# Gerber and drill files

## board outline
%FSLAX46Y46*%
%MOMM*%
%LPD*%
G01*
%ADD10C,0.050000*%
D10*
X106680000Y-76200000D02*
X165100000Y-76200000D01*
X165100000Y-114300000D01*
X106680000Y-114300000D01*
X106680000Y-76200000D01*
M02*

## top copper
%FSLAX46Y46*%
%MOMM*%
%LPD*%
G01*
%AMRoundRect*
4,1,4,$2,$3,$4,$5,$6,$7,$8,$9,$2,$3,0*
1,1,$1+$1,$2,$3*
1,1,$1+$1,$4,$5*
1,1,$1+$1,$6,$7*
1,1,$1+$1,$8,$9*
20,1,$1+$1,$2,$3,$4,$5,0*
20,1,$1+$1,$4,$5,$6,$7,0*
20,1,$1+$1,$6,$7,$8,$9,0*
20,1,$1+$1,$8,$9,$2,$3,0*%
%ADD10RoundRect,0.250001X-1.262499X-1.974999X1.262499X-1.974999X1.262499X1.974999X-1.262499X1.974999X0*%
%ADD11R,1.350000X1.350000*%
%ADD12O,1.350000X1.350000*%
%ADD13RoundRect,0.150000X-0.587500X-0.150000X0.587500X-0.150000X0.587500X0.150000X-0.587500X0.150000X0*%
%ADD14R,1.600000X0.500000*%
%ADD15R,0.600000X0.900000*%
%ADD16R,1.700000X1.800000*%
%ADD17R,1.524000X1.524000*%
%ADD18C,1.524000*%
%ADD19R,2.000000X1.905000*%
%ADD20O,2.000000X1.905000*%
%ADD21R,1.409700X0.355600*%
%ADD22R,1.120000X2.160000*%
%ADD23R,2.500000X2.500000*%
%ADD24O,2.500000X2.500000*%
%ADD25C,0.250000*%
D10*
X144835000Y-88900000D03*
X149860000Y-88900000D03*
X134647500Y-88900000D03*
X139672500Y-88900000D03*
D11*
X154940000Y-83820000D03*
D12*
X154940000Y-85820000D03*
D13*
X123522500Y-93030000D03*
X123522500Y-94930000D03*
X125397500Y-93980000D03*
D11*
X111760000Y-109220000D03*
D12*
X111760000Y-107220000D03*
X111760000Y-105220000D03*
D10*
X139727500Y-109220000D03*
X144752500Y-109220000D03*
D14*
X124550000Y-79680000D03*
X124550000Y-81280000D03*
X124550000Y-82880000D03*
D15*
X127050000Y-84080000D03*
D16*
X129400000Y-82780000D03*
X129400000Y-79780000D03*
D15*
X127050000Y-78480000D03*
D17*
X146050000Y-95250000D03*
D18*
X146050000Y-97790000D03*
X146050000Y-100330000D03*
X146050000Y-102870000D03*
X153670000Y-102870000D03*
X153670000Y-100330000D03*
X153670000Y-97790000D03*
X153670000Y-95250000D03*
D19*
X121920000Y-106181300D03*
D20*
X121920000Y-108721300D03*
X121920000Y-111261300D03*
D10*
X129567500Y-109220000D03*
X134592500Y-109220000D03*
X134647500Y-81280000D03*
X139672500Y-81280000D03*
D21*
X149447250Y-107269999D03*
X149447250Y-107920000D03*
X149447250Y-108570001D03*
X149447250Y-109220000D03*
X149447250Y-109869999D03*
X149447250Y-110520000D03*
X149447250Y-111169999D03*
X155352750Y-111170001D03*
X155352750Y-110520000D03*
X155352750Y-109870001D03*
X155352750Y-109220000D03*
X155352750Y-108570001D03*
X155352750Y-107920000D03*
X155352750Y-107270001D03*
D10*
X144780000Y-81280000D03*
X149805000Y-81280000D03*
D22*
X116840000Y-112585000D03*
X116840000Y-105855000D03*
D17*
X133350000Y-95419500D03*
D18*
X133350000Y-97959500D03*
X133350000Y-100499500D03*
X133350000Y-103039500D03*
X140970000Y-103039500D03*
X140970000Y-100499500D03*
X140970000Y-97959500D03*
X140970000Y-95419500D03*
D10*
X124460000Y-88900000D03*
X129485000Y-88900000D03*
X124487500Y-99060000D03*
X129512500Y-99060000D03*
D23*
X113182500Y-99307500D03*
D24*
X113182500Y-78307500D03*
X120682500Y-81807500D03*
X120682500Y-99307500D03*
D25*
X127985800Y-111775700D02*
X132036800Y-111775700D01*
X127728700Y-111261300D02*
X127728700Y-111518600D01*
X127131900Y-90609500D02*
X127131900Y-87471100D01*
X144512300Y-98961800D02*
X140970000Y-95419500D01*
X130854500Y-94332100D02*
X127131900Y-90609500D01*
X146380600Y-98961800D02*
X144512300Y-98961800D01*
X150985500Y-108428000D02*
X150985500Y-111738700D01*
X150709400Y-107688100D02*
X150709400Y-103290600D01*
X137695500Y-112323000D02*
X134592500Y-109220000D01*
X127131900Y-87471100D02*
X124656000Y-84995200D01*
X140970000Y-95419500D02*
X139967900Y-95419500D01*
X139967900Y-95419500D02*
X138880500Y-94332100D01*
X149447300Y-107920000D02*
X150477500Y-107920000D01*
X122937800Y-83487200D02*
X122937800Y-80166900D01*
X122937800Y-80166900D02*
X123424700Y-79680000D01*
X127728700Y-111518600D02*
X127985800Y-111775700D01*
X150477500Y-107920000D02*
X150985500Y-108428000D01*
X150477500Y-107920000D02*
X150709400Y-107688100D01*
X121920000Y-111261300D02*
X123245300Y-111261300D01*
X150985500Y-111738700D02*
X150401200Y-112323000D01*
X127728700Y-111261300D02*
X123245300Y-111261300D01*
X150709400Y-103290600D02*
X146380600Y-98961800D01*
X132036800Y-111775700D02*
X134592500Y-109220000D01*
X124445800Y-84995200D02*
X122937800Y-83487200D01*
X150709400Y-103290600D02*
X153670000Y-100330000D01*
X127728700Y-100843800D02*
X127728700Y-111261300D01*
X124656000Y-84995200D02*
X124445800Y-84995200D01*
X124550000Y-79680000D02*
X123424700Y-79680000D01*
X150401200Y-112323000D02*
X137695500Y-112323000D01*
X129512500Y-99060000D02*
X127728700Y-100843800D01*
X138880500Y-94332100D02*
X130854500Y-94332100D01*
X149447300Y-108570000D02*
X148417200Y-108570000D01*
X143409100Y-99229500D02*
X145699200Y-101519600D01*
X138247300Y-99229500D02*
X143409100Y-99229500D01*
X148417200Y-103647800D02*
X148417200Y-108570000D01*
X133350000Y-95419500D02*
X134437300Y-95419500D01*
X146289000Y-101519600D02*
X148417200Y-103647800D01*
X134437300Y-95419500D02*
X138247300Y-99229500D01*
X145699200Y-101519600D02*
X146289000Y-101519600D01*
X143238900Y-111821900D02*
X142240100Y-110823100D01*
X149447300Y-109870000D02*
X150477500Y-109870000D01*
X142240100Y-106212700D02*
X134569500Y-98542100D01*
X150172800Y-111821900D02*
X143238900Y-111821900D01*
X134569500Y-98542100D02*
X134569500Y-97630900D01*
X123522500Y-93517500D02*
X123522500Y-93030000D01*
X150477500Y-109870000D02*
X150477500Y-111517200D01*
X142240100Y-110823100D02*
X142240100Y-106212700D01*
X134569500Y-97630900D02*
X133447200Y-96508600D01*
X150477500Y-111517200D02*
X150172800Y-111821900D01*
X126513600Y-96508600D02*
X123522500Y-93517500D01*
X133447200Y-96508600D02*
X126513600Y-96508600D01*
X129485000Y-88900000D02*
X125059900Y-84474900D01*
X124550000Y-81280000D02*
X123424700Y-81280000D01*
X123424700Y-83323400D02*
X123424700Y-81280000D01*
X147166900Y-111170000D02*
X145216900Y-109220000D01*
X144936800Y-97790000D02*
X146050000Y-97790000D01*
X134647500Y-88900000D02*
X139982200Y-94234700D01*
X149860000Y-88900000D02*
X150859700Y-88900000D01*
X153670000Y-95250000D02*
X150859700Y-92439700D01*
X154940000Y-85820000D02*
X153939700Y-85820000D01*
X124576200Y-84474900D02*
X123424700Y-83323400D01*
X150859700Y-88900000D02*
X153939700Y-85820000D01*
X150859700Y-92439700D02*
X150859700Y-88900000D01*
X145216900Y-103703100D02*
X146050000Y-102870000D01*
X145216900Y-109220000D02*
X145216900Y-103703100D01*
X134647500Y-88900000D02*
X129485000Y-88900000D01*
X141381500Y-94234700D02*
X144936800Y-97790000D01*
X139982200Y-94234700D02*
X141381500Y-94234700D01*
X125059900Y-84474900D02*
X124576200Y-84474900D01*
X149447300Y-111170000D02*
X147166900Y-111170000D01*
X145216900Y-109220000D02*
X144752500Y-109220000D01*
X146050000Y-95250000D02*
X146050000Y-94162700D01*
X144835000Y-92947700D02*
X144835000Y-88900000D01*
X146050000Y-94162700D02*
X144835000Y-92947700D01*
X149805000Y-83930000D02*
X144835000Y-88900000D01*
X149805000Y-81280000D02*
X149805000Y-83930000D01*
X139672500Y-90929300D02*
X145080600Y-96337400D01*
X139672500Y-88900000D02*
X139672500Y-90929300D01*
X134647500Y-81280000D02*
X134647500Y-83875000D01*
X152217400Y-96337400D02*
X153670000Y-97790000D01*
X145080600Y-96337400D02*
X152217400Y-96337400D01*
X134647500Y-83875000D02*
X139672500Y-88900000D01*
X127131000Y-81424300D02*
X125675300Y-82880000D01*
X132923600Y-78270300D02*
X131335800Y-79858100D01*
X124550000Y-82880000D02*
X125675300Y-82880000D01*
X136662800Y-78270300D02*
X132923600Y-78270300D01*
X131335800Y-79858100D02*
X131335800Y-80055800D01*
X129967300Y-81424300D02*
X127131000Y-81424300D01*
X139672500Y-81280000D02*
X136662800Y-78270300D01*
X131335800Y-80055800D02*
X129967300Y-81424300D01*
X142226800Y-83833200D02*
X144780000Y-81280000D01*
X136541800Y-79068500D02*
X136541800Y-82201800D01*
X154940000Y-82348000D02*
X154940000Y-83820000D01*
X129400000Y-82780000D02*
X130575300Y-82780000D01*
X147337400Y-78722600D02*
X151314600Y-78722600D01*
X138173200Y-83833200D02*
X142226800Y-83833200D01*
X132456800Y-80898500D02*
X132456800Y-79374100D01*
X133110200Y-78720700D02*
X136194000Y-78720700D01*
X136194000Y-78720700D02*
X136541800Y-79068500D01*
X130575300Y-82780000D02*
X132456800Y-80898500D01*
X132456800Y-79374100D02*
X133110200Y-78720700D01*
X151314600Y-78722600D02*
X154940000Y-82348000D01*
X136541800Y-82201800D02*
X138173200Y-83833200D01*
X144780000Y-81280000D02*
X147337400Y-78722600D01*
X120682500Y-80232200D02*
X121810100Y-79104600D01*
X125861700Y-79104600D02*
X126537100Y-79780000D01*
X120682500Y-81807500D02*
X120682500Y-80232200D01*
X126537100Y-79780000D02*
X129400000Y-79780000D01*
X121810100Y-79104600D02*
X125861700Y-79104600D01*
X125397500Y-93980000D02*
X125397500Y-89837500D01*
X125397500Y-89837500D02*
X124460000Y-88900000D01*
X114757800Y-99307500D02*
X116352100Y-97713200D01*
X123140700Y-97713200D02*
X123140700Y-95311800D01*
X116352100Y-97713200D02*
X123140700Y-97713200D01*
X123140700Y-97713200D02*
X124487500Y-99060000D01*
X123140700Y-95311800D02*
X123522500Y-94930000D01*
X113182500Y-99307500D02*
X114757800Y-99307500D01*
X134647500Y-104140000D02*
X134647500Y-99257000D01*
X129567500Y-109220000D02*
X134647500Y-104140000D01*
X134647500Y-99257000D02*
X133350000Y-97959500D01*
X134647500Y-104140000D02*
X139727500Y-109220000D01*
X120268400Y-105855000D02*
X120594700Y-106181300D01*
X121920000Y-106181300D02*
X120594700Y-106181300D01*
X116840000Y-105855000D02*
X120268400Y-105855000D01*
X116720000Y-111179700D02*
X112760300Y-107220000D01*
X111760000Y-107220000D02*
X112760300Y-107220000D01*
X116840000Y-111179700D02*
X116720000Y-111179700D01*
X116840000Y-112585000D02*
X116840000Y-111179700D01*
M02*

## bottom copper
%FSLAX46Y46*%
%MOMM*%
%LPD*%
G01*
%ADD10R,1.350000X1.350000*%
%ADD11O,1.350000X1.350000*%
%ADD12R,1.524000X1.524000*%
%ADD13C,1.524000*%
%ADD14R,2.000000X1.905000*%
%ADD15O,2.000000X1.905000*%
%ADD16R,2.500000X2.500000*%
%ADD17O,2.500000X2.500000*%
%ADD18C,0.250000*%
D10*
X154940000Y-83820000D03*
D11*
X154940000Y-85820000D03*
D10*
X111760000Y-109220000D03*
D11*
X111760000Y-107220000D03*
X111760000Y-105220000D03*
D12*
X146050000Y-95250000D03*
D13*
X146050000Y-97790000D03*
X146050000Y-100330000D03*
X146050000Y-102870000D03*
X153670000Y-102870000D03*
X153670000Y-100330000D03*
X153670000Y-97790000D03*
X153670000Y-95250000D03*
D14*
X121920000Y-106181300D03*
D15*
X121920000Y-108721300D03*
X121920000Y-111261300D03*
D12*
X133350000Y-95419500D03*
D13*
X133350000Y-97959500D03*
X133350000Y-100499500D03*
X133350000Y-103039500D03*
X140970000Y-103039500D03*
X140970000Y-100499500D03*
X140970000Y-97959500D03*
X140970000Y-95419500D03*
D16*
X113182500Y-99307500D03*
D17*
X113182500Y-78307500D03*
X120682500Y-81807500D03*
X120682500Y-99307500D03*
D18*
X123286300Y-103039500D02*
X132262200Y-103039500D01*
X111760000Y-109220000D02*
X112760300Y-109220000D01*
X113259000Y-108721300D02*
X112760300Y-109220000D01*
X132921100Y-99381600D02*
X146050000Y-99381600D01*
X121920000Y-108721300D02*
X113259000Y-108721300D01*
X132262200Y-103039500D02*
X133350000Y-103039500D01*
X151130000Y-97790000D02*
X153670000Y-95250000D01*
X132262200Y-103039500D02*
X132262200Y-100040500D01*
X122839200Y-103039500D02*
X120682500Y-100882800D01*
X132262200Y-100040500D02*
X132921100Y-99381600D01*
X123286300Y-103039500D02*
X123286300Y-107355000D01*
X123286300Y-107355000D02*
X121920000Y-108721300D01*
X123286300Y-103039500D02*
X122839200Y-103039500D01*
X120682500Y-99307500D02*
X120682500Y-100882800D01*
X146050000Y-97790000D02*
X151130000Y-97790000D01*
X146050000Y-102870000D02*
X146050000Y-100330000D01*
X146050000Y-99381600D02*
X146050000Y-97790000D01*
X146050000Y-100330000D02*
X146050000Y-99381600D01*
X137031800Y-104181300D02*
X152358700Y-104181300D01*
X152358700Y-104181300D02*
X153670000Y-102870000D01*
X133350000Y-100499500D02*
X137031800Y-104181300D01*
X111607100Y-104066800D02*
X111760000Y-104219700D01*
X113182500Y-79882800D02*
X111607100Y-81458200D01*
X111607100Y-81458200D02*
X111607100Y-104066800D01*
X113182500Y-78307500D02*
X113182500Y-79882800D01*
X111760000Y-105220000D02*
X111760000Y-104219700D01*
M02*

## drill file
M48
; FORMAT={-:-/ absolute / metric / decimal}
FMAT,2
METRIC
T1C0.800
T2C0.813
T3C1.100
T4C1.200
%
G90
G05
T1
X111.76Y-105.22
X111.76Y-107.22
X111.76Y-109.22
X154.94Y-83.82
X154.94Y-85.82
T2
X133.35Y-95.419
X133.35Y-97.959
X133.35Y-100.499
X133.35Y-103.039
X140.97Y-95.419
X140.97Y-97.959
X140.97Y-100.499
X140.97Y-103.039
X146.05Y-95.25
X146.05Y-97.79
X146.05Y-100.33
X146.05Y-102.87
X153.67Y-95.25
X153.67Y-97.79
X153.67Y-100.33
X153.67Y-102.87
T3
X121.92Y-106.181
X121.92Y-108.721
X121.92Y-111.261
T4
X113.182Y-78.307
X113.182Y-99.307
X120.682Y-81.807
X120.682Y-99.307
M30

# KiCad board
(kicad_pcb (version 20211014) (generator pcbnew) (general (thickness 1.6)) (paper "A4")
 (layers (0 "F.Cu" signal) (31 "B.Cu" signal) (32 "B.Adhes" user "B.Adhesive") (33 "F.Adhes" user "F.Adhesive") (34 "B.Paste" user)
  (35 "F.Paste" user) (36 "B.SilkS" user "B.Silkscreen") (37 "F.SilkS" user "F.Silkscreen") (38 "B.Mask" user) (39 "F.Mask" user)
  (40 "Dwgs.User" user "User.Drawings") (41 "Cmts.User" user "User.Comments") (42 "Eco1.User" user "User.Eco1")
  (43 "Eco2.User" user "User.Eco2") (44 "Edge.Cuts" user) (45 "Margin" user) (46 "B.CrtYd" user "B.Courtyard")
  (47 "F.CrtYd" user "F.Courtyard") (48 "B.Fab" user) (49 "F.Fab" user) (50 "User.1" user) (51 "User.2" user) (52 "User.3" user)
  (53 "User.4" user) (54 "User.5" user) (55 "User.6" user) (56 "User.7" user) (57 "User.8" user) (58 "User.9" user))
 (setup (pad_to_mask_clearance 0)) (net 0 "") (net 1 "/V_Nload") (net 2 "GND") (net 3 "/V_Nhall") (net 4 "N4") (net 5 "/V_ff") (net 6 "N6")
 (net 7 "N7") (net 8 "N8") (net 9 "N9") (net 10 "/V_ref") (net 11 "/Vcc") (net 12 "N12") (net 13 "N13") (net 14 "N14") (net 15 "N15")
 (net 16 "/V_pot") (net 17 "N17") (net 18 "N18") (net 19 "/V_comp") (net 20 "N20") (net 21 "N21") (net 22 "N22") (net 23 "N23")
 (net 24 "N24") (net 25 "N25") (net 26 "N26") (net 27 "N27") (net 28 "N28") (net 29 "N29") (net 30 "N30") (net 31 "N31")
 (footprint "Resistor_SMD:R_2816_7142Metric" (layer "F.Cu") (at 147.3475 88.9)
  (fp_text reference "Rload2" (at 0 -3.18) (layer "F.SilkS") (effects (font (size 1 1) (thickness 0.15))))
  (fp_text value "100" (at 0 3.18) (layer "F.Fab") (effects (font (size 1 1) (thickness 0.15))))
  (pad "1" smd roundrect (at -2.5125 0) (size 3.025 4.45) (layers "F.Cu" "F.Paste" "F.Mask") (roundrect_rratio 0.08264495868)
   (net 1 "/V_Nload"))
  (pad "2" smd roundrect (at 2.5125 0) (size 3.025 4.45) (layers "F.Cu" "F.Paste" "F.Mask") (roundrect_rratio 0.08264495868) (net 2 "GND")))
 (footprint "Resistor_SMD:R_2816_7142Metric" (layer "F.Cu") (at 137.16 88.9)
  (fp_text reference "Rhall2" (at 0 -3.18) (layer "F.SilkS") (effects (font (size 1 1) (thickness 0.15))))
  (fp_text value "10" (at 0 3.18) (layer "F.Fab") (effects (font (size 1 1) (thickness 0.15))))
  (pad "1" smd roundrect (at -2.5125 0) (size 3.025 4.45) (layers "F.Cu" "F.Paste" "F.Mask") (roundrect_rratio 0.08264495868) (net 2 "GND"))
  (pad "2" smd roundrect (at 2.5125 0) (size 3.025 4.45) (layers "F.Cu" "F.Paste" "F.Mask") (roundrect_rratio 0.08264495868)
   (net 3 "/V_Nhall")))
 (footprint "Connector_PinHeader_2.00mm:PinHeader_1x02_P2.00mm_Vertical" (layer "F.Cu") (at 154.94 83.82)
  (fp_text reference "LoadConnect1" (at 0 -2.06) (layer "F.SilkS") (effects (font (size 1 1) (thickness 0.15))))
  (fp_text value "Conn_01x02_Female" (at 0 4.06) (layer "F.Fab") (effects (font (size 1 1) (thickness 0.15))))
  (pad "1" thru_hole rect (at 0 0) (size 1.35 1.35) (drill 0.8) (layers *.Cu *.Mask) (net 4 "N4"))
  (pad "2" thru_hole oval (at 0 2) (size 1.35 1.35) (drill 0.8) (layers *.Cu *.Mask) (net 2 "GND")))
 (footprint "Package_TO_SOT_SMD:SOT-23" (layer "F.Cu") (at 124.46 93.98)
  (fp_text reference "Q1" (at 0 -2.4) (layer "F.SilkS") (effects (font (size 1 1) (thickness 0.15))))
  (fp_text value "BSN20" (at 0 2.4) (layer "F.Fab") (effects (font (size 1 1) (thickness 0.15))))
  (pad "1" smd roundrect (at -0.9375 -0.95) (size 1.475 0.6) (layers "F.Cu" "F.Paste" "F.Mask") (roundrect_rratio 0.25) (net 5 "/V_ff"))
  (pad "2" smd roundrect (at -0.9375 0.95) (size 1.475 0.6) (layers "F.Cu" "F.Paste" "F.Mask") (roundrect_rratio 0.25) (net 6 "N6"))
  (pad "3" smd roundrect (at 0.9375 0) (size 1.475 0.6) (layers "F.Cu" "F.Paste" "F.Mask") (roundrect_rratio 0.25) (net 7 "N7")))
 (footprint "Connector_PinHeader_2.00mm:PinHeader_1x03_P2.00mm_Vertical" (layer "F.Cu") (at 111.76 109.22 180)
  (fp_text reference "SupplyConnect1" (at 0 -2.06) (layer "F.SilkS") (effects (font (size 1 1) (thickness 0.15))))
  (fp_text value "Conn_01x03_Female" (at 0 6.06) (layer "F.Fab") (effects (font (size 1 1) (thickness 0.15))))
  (pad "1" thru_hole rect (at 0 0 180) (size 1.35 1.35) (drill 0.8) (layers *.Cu *.Mask) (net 2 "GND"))
  (pad "2" thru_hole oval (at 0 2 180) (size 1.35 1.35) (drill 0.8) (layers *.Cu *.Mask) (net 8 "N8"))
  (pad "3" thru_hole oval (at 0 4 180) (size 1.35 1.35) (drill 0.8) (layers *.Cu *.Mask) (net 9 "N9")))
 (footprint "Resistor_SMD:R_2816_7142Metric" (layer "F.Cu") (at 142.24 109.22)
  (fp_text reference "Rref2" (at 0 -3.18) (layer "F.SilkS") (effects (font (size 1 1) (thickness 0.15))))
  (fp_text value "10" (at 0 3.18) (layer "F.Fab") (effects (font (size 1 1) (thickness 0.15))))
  (pad "1" smd roundrect (at -2.5125 0) (size 3.025 4.45) (layers "F.Cu" "F.Paste" "F.Mask") (roundrect_rratio 0.08264495868)
   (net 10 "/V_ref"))
  (pad "2" smd roundrect (at 2.5125 0) (size 3.025 4.45) (layers "F.Cu" "F.Paste" "F.Mask") (roundrect_rratio 0.08264495868) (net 2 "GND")))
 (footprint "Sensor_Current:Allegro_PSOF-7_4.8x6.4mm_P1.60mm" (layer "F.Cu") (at 127 81.28)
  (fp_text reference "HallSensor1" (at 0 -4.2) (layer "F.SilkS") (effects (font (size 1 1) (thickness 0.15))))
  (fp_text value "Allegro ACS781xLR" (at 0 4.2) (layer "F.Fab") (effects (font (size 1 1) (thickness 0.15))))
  (pad "1" smd rect (at -2.45 -1.6) (size 1.6 0.5) (layers "F.Cu" "F.Paste" "F.Mask") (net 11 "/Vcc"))
  (pad "2" smd rect (at -2.45 0) (size 1.6 0.5) (layers "F.Cu" "F.Paste" "F.Mask") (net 2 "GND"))
  (pad "3" smd rect (at -2.45 1.6) (size 1.6 0.5) (layers "F.Cu" "F.Paste" "F.Mask") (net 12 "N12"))
  (pad "4" smd rect (at 0.05 2.8) (size 0.6 0.9) (layers "F.Cu" "F.Paste" "F.Mask") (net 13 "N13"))
  (pad "5" smd rect (at 2.4 1.5) (size 1.7 1.8) (layers "F.Cu" "F.Paste" "F.Mask") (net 4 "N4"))
  (pad "6" smd rect (at 2.4 -1.5) (size 1.7 1.8) (layers "F.Cu" "F.Paste" "F.Mask") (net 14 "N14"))
  (pad "7" smd rect (at 0.05 -2.8) (size 0.6 0.9) (layers "F.Cu" "F.Paste" "F.Mask") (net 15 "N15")))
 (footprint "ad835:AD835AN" (layer "F.Cu") (at 146.05 95.25)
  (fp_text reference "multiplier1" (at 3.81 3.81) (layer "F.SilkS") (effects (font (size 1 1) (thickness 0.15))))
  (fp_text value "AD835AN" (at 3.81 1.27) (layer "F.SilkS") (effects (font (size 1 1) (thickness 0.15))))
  (pad "1" thru_hole rect locked (at 0 0) (size 1.524 1.524) (drill 0.8128) (layers *.Cu *.Mask) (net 1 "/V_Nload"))
  (pad "2" thru_hole circle locked (at 0 2.54) (size 1.524 1.524) (drill 0.8128) (layers *.Cu *.Mask) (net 2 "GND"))
  (pad "3" thru_hole circle locked (at 0 5.08) (size 1.524 1.524) (drill 0.8128) (layers *.Cu *.Mask) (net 2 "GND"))
  (pad "4" thru_hole circle locked (at 0 7.62) (size 1.524 1.524) (drill 0.8128) (layers *.Cu *.Mask) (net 2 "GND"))
  (pad "5" thru_hole circle locked (at 7.62 7.62) (size 1.524 1.524) (drill 0.8128) (layers *.Cu *.Mask) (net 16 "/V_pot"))
  (pad "6" thru_hole circle locked (at 7.62 5.08) (size 1.524 1.524) (drill 0.8128) (layers *.Cu *.Mask) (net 11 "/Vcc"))
  (pad "7" thru_hole circle locked (at 7.62 2.54) (size 1.524 1.524) (drill 0.8128) (layers *.Cu *.Mask) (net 3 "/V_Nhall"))
  (pad "8" thru_hole circle locked (at 7.62 0) (size 1.524 1.524) (drill 0.8128) (layers *.Cu *.Mask) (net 2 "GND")))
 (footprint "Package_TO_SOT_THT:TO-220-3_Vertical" (layer "F.Cu") (at 121.92 106.1813 -90)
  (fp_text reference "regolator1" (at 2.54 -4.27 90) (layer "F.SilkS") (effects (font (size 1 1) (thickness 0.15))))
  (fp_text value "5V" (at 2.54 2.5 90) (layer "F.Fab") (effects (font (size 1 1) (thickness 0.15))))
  (pad "1" thru_hole rect (at 0 0 270) (size 1.905 2) (drill 1.1) (layers *.Cu *.Mask) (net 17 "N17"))
  (pad "2" thru_hole oval (at 2.54 0 270) (size 1.905 2) (drill 1.1) (layers *.Cu *.Mask) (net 2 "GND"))
  (pad "3" thru_hole oval (at 5.08 0 270) (size 1.905 2) (drill 1.1) (layers *.Cu *.Mask) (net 11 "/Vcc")))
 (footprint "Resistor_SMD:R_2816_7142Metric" (layer "F.Cu") (at 132.08 109.22)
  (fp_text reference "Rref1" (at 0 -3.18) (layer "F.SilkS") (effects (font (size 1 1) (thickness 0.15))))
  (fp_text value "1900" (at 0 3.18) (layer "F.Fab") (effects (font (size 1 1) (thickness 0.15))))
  (pad "1" smd roundrect (at -2.5125 0) (size 3.025 4.45) (layers "F.Cu" "F.Paste" "F.Mask") (roundrect_rratio 0.08264495868)
   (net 10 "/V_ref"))
  (pad "2" smd roundrect (at 2.5125 0) (size 3.025 4.45) (layers "F.Cu" "F.Paste" "F.Mask") (roundrect_rratio 0.08264495868) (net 11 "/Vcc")))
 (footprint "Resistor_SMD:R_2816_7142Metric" (layer "F.Cu") (at 137.16 81.28)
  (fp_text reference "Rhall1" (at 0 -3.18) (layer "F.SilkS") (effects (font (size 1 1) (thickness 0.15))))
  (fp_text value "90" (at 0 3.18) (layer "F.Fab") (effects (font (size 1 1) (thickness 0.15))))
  (pad "1" smd roundrect (at -2.5125 0) (size 3.025 4.45) (layers "F.Cu" "F.Paste" "F.Mask") (roundrect_rratio 0.08264495868)
   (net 3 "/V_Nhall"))
  (pad "2" smd roundrect (at 2.5125 0) (size 3.025 4.45) (layers "F.Cu" "F.Paste" "F.Mask") (roundrect_rratio 0.08264495868) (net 12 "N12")))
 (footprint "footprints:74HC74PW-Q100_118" (layer "F.Cu") (at 152.4 109.22)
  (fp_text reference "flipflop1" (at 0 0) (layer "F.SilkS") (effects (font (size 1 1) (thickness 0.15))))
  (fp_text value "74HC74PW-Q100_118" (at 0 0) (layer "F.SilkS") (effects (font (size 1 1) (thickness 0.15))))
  (pad "1" smd rect locked (at -2.95275 -1.950001) (size 1.4097 0.3556) (layers "F.Cu" "F.Paste" "F.Mask") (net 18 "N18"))
  (pad "2" smd rect locked (at -2.95275 -1.3) (size 1.4097 0.3556) (layers "F.Cu" "F.Paste" "F.Mask") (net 11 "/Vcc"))
  (pad "3" smd rect locked (at -2.95275 -0.649999) (size 1.4097 0.3556) (layers "F.Cu" "F.Paste" "F.Mask") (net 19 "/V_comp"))
  (pad "4" smd rect locked (at -2.95275 0) (size 1.4097 0.3556) (layers "F.Cu" "F.Paste" "F.Mask") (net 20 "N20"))
  (pad "5" smd rect locked (at -2.95275 0.649999) (size 1.4097 0.3556) (layers "F.Cu" "F.Paste" "F.Mask") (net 5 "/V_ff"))
  (pad "6" smd rect locked (at -2.95275 1.3) (size 1.4097 0.3556) (layers "F.Cu" "F.Paste" "F.Mask") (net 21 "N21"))
  (pad "7" smd rect locked (at -2.95275 1.949999) (size 1.4097 0.3556) (layers "F.Cu" "F.Paste" "F.Mask") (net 2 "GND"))
  (pad "8" smd rect locked (at 2.95275 1.950001) (size 1.4097 0.3556) (layers "F.Cu" "F.Paste" "F.Mask") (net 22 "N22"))
  (pad "9" smd rect locked (at 2.95275 1.3) (size 1.4097 0.3556) (layers "F.Cu" "F.Paste" "F.Mask") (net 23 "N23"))
  (pad "10" smd rect locked (at 2.95275 0.650001) (size 1.4097 0.3556) (layers "F.Cu" "F.Paste" "F.Mask") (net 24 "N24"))
  (pad "11" smd rect locked (at 2.95275 0) (size 1.4097 0.3556) (layers "F.Cu" "F.Paste" "F.Mask") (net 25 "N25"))
  (pad "12" smd rect locked (at 2.95275 -0.649999) (size 1.4097 0.3556) (layers "F.Cu" "F.Paste" "F.Mask") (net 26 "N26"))
  (pad "13" smd rect locked (at 2.95275 -1.3) (size 1.4097 0.3556) (layers "F.Cu" "F.Paste" "F.Mask") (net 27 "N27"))
  (pad "14" smd rect locked (at 2.95275 -1.949999) (size 1.4097 0.3556) (layers "F.Cu" "F.Paste" "F.Mask") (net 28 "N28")))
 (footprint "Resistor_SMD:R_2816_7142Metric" (layer "F.Cu") (at 147.2925 81.28)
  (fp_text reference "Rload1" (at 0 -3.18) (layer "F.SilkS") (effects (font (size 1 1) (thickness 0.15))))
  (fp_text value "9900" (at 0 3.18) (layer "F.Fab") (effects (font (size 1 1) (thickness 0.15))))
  (pad "1" smd roundrect (at -2.5125 0) (size 3.025 4.45) (layers "F.Cu" "F.Paste" "F.Mask") (roundrect_rratio 0.08264495868) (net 4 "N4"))
  (pad "2" smd roundrect (at 2.5125 0) (size 3.025 4.45) (layers "F.Cu" "F.Paste" "F.Mask") (roundrect_rratio 0.08264495868)
   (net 1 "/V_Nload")))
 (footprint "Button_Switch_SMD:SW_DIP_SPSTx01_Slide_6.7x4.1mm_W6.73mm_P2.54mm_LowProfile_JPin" (layer "F.Cu") (at 116.84 109.22 90)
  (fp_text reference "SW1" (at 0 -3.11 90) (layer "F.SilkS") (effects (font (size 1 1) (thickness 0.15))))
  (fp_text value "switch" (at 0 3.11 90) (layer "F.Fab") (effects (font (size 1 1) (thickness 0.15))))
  (pad "1" smd rect (at -3.365 0 90) (size 2.16 1.12) (layers "F.Cu" "F.Paste" "F.Mask") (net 8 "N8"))
  (pad "2" smd rect (at 3.365 0 90) (size 2.16 1.12) (layers "F.Cu" "F.Paste" "F.Mask") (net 17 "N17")))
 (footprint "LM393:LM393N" (layer "F.Cu") (at 133.35 95.4195)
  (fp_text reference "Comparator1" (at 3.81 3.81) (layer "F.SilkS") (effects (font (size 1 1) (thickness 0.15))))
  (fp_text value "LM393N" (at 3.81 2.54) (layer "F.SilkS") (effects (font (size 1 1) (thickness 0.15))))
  (pad "1" thru_hole rect locked (at 0 0) (size 1.524 1.524) (drill 0.8128) (layers *.Cu *.Mask) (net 19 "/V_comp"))
  (pad "2" thru_hole circle locked (at 0 2.54) (size 1.524 1.524) (drill 0.8128) (layers *.Cu *.Mask) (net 10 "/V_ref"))
  (pad "3" thru_hole circle locked (at 0 5.08) (size 1.524 1.524) (drill 0.8128) (layers *.Cu *.Mask) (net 16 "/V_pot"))
  (pad "4" thru_hole circle locked (at 0 7.62) (size 1.524 1.524) (drill 0.8128) (layers *.Cu *.Mask) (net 2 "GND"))
  (pad "5" thru_hole circle locked (at 7.62 7.62) (size 1.524 1.524) (drill 0.8128) (layers *.Cu *.Mask) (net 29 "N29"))
  (pad "6" thru_hole circle locked (at 7.62 5.08) (size 1.524 1.524) (drill 0.8128) (layers *.Cu *.Mask) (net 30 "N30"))
  (pad "7" thru_hole circle locked (at 7.62 2.54) (size 1.524 1.524) (drill 0.8128) (layers *.Cu *.Mask) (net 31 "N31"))
  (pad "8" thru_hole circle locked (at 7.62 0) (size 1.524 1.524) (drill 0.8128) (layers *.Cu *.Mask) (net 11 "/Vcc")))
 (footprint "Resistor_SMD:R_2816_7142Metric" (layer "F.Cu") (at 126.9725 88.9)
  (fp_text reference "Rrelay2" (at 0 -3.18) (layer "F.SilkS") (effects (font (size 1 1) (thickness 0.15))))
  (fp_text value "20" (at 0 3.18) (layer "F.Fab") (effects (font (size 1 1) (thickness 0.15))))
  (pad "1" smd roundrect (at -2.5125 0) (size 3.025 4.45) (layers "F.Cu" "F.Paste" "F.Mask") (roundrect_rratio 0.08264495868) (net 7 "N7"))
  (pad "2" smd roundrect (at 2.5125 0) (size 3.025 4.45) (layers "F.Cu" "F.Paste" "F.Mask") (roundrect_rratio 0.08264495868) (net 2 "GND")))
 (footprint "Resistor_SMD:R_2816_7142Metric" (layer "F.Cu") (at 127 99.06)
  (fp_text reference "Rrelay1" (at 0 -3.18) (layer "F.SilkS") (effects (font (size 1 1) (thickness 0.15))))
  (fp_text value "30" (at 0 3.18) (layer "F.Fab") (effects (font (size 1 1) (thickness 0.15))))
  (pad "1" smd roundrect (at -2.5125 0) (size 3.025 4.45) (layers "F.Cu" "F.Paste" "F.Mask") (roundrect_rratio 0.08264495868) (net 6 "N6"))
  (pad "2" smd roundrect (at 2.5125 0) (size 3.025 4.45) (layers "F.Cu" "F.Paste" "F.Mask") (roundrect_rratio 0.08264495868) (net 11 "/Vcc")))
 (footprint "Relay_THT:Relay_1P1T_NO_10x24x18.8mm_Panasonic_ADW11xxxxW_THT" (layer "B.Cu") (at 113.1825 99.3075)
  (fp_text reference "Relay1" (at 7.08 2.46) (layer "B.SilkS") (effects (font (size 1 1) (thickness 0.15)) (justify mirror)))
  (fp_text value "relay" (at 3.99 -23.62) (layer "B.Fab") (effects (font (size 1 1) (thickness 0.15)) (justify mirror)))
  (pad "1" thru_hole rect (at 0 0) (size 2.5 2.5) (drill 1.2) (layers *.Cu *.Mask) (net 6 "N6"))
  (pad "3" thru_hole oval (at 0 -21) (size 2.5 2.5) (drill 1.2) (layers *.Cu *.Mask) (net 9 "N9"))
  (pad "5" thru_hole oval (at 7.5 -17.5) (size 2.5 2.5) (drill 1.2) (layers *.Cu *.Mask) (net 14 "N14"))
  (pad "6" thru_hole oval (at 7.5 0) (size 2.5 2.5) (drill 1.2) (layers *.Cu *.Mask) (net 2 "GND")))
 (gr_rect (start 106.68 114.3) (end 165.1 76.2) (layer "Edge.Cuts") (width 0.05) (fill none))
 (segment (start 127.9858 111.7757) (end 132.0368 111.7757) (width 0.25) (layer "F.Cu") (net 11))
 (segment (start 127.7287 111.2613) (end 127.7287 111.5186) (width 0.25) (layer "F.Cu") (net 11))
 (segment (start 127.1319 90.6095) (end 127.1319 87.4711) (width 0.25) (layer "F.Cu") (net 11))
 (segment (start 144.5123 98.9618) (end 140.97 95.4195) (width 0.25) (layer "F.Cu") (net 11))
 (segment (start 130.8545 94.3321) (end 127.1319 90.6095) (width 0.25) (layer "F.Cu") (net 11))
 (segment (start 146.3806 98.9618) (end 144.5123 98.9618) (width 0.25) (layer "F.Cu") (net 11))
 (segment (start 150.9855 108.428) (end 150.9855 111.7387) (width 0.25) (layer "F.Cu") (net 11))
 (segment (start 150.7094 107.6881) (end 150.7094 103.2906) (width 0.25) (layer "F.Cu") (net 11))
 (segment (start 137.6955 112.323) (end 134.5925 109.22) (width 0.25) (layer "F.Cu") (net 11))
 (segment (start 127.1319 87.4711) (end 124.656 84.9952) (width 0.25) (layer "F.Cu") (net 11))
 (segment (start 140.97 95.4195) (end 139.9679 95.4195) (width 0.25) (layer "F.Cu") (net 11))
 (segment (start 139.9679 95.4195) (end 138.8805 94.3321) (width 0.25) (layer "F.Cu") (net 11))
 (segment (start 149.4473 107.92) (end 150.4775 107.92) (width 0.25) (layer "F.Cu") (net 11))
 (segment (start 122.9378 83.4872) (end 122.9378 80.1669) (width 0.25) (layer "F.Cu") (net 11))
 (segment (start 122.9378 80.1669) (end 123.4247 79.68) (width 0.25) (layer "F.Cu") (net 11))
 (segment (start 127.7287 111.5186) (end 127.9858 111.7757) (width 0.25) (layer "F.Cu") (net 11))
 (segment (start 150.4775 107.92) (end 150.9855 108.428) (width 0.25) (layer "F.Cu") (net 11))
 (segment (start 150.4775 107.92) (end 150.7094 107.6881) (width 0.25) (layer "F.Cu") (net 11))
 (segment (start 121.92 111.2613) (end 123.2453 111.2613) (width 0.25) (layer "F.Cu") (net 11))
 (segment (start 150.9855 111.7387) (end 150.4012 112.323) (width 0.25) (layer "F.Cu") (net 11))
 (segment (start 127.7287 111.2613) (end 123.2453 111.2613) (width 0.25) (layer "F.Cu") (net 11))
 (segment (start 150.7094 103.2906) (end 146.3806 98.9618) (width 0.25) (layer "F.Cu") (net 11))
 (segment (start 132.0368 111.7757) (end 134.5925 109.22) (width 0.25) (layer "F.Cu") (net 11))
 (segment (start 124.4458 84.9952) (end 122.9378 83.4872) (width 0.25) (layer "F.Cu") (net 11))
 (segment (start 150.7094 103.2906) (end 153.67 100.33) (width 0.25) (layer "F.Cu") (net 11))
 (segment (start 127.7287 100.8438) (end 127.7287 111.2613) (width 0.25) (layer "F.Cu") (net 11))
 (segment (start 124.656 84.9952) (end 124.4458 84.9952) (width 0.25) (layer "F.Cu") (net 11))
 (segment (start 124.55 79.68) (end 123.4247 79.68) (width 0.25) (layer "F.Cu") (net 11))
 (segment (start 150.4012 112.323) (end 137.6955 112.323) (width 0.25) (layer "F.Cu") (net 11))
 (segment (start 129.5125 99.06) (end 127.7287 100.8438) (width 0.25) (layer "F.Cu") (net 11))
 (segment (start 138.8805 94.3321) (end 130.8545 94.3321) (width 0.25) (layer "F.Cu") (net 11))
 (segment (start 149.4473 108.57) (end 148.4172 108.57) (width 0.25) (layer "F.Cu") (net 19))
 (segment (start 143.4091 99.2295) (end 145.6992 101.5196) (width 0.25) (layer "F.Cu") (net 19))
 (segment (start 138.2473 99.2295) (end 143.4091 99.2295) (width 0.25) (layer "F.Cu") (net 19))
 (segment (start 148.4172 103.6478) (end 148.4172 108.57) (width 0.25) (layer "F.Cu") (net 19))
 (segment (start 133.35 95.4195) (end 134.4373 95.4195) (width 0.25) (layer "F.Cu") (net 19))
 (segment (start 146.289 101.5196) (end 148.4172 103.6478) (width 0.25) (layer "F.Cu") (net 19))
 (segment (start 134.4373 95.4195) (end 138.2473 99.2295) (width 0.25) (layer "F.Cu") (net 19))
 (segment (start 145.6992 101.5196) (end 146.289 101.5196) (width 0.25) (layer "F.Cu") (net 19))
 (segment (start 143.2389 111.8219) (end 142.2401 110.8231) (width 0.25) (layer "F.Cu") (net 5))
 (segment (start 149.4473 109.87) (end 150.4775 109.87) (width 0.25) (layer "F.Cu") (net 5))
 (segment (start 142.2401 106.2127) (end 134.5695 98.5421) (width 0.25) (layer "F.Cu") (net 5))
 (segment (start 150.1728 111.8219) (end 143.2389 111.8219) (width 0.25) (layer "F.Cu") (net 5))
 (segment (start 134.5695 98.5421) (end 134.5695 97.6309) (width 0.25) (layer "F.Cu") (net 5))
 (segment (start 123.5225 93.5175) (end 123.5225 93.03) (width 0.25) (layer "F.Cu") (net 5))
 (segment (start 150.4775 109.87) (end 150.4775 111.5172) (width 0.25) (layer "F.Cu") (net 5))
 (segment (start 142.2401 110.8231) (end 142.2401 106.2127) (width 0.25) (layer "F.Cu") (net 5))
 (segment (start 134.5695 97.6309) (end 133.4472 96.5086) (width 0.25) (layer "F.Cu") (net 5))
 (segment (start 150.4775 111.5172) (end 150.1728 111.8219) (width 0.25) (layer "F.Cu") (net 5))
 (segment (start 126.5136 96.5086) (end 123.5225 93.5175) (width 0.25) (layer "F.Cu") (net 5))
 (segment (start 133.4472 96.5086) (end 126.5136 96.5086) (width 0.25) (layer "F.Cu") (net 5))
 (segment (start 129.485 88.9) (end 125.0599 84.4749) (width 0.25) (layer "F.Cu") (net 2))
 (segment (start 124.55 81.28) (end 123.4247 81.28) (width 0.25) (layer "F.Cu") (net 2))
 (segment (start 123.4247 83.3234) (end 123.4247 81.28) (width 0.25) (layer "F.Cu") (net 2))
 (segment (start 147.1669 111.17) (end 145.2169 109.22) (width 0.25) (layer "F.Cu") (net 2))
 (segment (start 144.9368 97.79) (end 146.05 97.79) (width 0.25) (layer "F.Cu") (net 2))
 (segment (start 134.6475 88.9) (end 139.9822 94.2347) (width 0.25) (layer "F.Cu") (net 2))
 (segment (start 149.86 88.9) (end 150.8597 88.9) (width 0.25) (layer "F.Cu") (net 2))
 (segment (start 153.67 95.25) (end 150.8597 92.4397) (width 0.25) (layer "F.Cu") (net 2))
 (segment (start 154.94 85.82) (end 153.9397 85.82) (width 0.25) (layer "F.Cu") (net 2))
 (segment (start 124.5762 84.4749) (end 123.4247 83.3234) (width 0.25) (layer "F.Cu") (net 2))
 (segment (start 150.8597 88.9) (end 153.9397 85.82) (width 0.25) (layer "F.Cu") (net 2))
 (segment (start 150.8597 92.4397) (end 150.8597 88.9) (width 0.25) (layer "F.Cu") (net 2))
 (segment (start 145.2169 103.7031) (end 146.05 102.87) (width 0.25) (layer "F.Cu") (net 2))
 (segment (start 145.2169 109.22) (end 145.2169 103.7031) (width 0.25) (layer "F.Cu") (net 2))
 (segment (start 134.6475 88.9) (end 129.485 88.9) (width 0.25) (layer "F.Cu") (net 2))
 (segment (start 141.3815 94.2347) (end 144.9368 97.79) (width 0.25) (layer "F.Cu") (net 2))
 (segment (start 139.9822 94.2347) (end 141.3815 94.2347) (width 0.25) (layer "F.Cu") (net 2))
 (segment (start 125.0599 84.4749) (end 124.5762 84.4749) (width 0.25) (layer "F.Cu") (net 2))
 (segment (start 149.4473 111.17) (end 147.1669 111.17) (width 0.25) (layer "F.Cu") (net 2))
 (segment (start 145.2169 109.22) (end 144.7525 109.22) (width 0.25) (layer "F.Cu") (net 2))
 (segment (start 123.2863 103.0395) (end 132.2622 103.0395) (width 0.25) (layer "B.Cu") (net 2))
 (segment (start 111.76 109.22) (end 112.7603 109.22) (width 0.25) (layer "B.Cu") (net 2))
 (segment (start 113.259 108.7213) (end 112.7603 109.22) (width 0.25) (layer "B.Cu") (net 2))
 (segment (start 132.9211 99.3816) (end 146.05 99.3816) (width 0.25) (layer "B.Cu") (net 2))
 (segment (start 121.92 108.7213) (end 113.259 108.7213) (width 0.25) (layer "B.Cu") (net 2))
 (segment (start 132.2622 103.0395) (end 133.35 103.0395) (width 0.25) (layer "B.Cu") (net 2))
 (segment (start 151.13 97.79) (end 153.67 95.25) (width 0.25) (layer "B.Cu") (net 2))
 (segment (start 132.2622 103.0395) (end 132.2622 100.0405) (width 0.25) (layer "B.Cu") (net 2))
 (segment (start 122.8392 103.0395) (end 120.6825 100.8828) (width 0.25) (layer "B.Cu") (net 2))
 (segment (start 132.2622 100.0405) (end 132.9211 99.3816) (width 0.25) (layer "B.Cu") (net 2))
 (segment (start 123.2863 103.0395) (end 123.2863 107.355) (width 0.25) (layer "B.Cu") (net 2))
 (segment (start 123.2863 107.355) (end 121.92 108.7213) (width 0.25) (layer "B.Cu") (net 2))
 (segment (start 123.2863 103.0395) (end 122.8392 103.0395) (width 0.25) (layer "B.Cu") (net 2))
 (segment (start 120.6825 99.3075) (end 120.6825 100.8828) (width 0.25) (layer "B.Cu") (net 2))
 (segment (start 146.05 97.79) (end 151.13 97.79) (width 0.25) (layer "B.Cu") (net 2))
 (segment (start 146.05 102.87) (end 146.05 100.33) (width 0.25) (layer "B.Cu") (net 2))
 (segment (start 146.05 99.3816) (end 146.05 97.79) (width 0.25) (layer "B.Cu") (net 2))
 (segment (start 146.05 100.33) (end 146.05 99.3816) (width 0.25) (layer "B.Cu") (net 2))
 (segment (start 146.05 95.25) (end 146.05 94.1627) (width 0.25) (layer "F.Cu") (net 1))
 (segment (start 144.835 92.9477) (end 144.835 88.9) (width 0.25) (layer "F.Cu") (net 1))
 (segment (start 146.05 94.1627) (end 144.835 92.9477) (width 0.25) (layer "F.Cu") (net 1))
 (segment (start 149.805 83.93) (end 144.835 88.9) (width 0.25) (layer "F.Cu") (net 1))
 (segment (start 149.805 81.28) (end 149.805 83.93) (width 0.25) (layer "F.Cu") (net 1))
 (segment (start 137.0318 104.1813) (end 152.3587 104.1813) (width 0.25) (layer "B.Cu") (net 16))
 (segment (start 152.3587 104.1813) (end 153.67 102.87) (width 0.25) (layer "B.Cu") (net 16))
 (segment (start 133.35 100.4995) (end 137.0318 104.1813) (width 0.25) (layer "B.Cu") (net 16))
 (segment (start 139.6725 90.9293) (end 145.0806 96.3374) (width 0.25) (layer "F.Cu") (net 3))
 (segment (start 139.6725 88.9) (end 139.6725 90.9293) (width 0.25) (layer "F.Cu") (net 3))
 (segment (start 134.6475 81.28) (end 134.6475 83.875) (width 0.25) (layer "F.Cu") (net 3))
 (segment (start 152.2174 96.3374) (end 153.67 97.79) (width 0.25) (layer "F.Cu") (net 3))
 (segment (start 145.0806 96.3374) (end 152.2174 96.3374) (width 0.25) (layer "F.Cu") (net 3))
 (segment (start 134.6475 83.875) (end 139.6725 88.9) (width 0.25) (layer "F.Cu") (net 3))
 (segment (start 127.131 81.4243) (end 125.6753 82.88) (width 0.25) (layer "F.Cu") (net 12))
 (segment (start 132.9236 78.2703) (end 131.3358 79.8581) (width 0.25) (layer "F.Cu") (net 12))
 (segment (start 124.55 82.88) (end 125.6753 82.88) (width 0.25) (layer "F.Cu") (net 12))
 (segment (start 136.6628 78.2703) (end 132.9236 78.2703) (width 0.25) (layer "F.Cu") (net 12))
 (segment (start 131.3358 79.8581) (end 131.3358 80.0558) (width 0.25) (layer "F.Cu") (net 12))
 (segment (start 129.9673 81.4243) (end 127.131 81.4243) (width 0.25) (layer "F.Cu") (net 12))
 (segment (start 139.6725 81.28) (end 136.6628 78.2703) (width 0.25) (layer "F.Cu") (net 12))
 (segment (start 131.3358 80.0558) (end 129.9673 81.4243) (width 0.25) (layer "F.Cu") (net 12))
 (segment (start 142.2268 83.8332) (end 144.78 81.28) (width 0.25) (layer "F.Cu") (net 4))
 (segment (start 136.5418 79.0685) (end 136.5418 82.2018) (width 0.25) (layer "F.Cu") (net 4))
 (segment (start 154.94 82.348) (end 154.94 83.82) (width 0.25) (layer "F.Cu") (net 4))
 (segment (start 129.4 82.78) (end 130.5753 82.78) (width 0.25) (layer "F.Cu") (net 4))
 (segment (start 147.3374 78.7226) (end 151.3146 78.7226) (width 0.25) (layer "F.Cu") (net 4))
 (segment (start 138.1732 83.8332) (end 142.2268 83.8332) (width 0.25) (layer "F.Cu") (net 4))
 (segment (start 132.4568 80.8985) (end 132.4568 79.3741) (width 0.25) (layer "F.Cu") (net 4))
 (segment (start 133.1102 78.7207) (end 136.194 78.7207) (width 0.25) (layer "F.Cu") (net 4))
 (segment (start 136.194 78.7207) (end 136.5418 79.0685) (width 0.25) (layer "F.Cu") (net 4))
 (segment (start 130.5753 82.78) (end 132.4568 80.8985) (width 0.25) (layer "F.Cu") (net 4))
 (segment (start 132.4568 79.3741) (end 133.1102 78.7207) (width 0.25) (layer "F.Cu") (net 4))
 (segment (start 151.3146 78.7226) (end 154.94 82.348) (width 0.25) (layer "F.Cu") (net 4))
 (segment (start 136.5418 82.2018) (end 138.1732 83.8332) (width 0.25) (layer "F.Cu") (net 4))
 (segment (start 144.78 81.28) (end 147.3374 78.7226) (width 0.25) (layer "F.Cu") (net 4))
 (segment (start 120.6825 80.2322) (end 121.8101 79.1046) (width 0.25) (layer "F.Cu") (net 14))
 (segment (start 125.8617 79.1046) (end 126.5371 79.78) (width 0.25) (layer "F.Cu") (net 14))
 (segment (start 120.6825 81.8075) (end 120.6825 80.2322) (width 0.25) (layer "F.Cu") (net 14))
 (segment (start 126.5371 79.78) (end 129.4 79.78) (width 0.25) (layer "F.Cu") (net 14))
 (segment (start 121.8101 79.1046) (end 125.8617 79.1046) (width 0.25) (layer "F.Cu") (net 14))
 (segment (start 125.3975 93.98) (end 125.3975 89.8375) (width 0.25) (layer "F.Cu") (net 7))
 (segment (start 125.3975 89.8375) (end 124.46 88.9) (width 0.25) (layer "F.Cu") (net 7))
 (segment (start 114.7578 99.3075) (end 116.3521 97.7132) (width 0.25) (layer "F.Cu") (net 6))
 (segment (start 123.1407 97.7132) (end 123.1407 95.3118) (width 0.25) (layer "F.Cu") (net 6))
 (segment (start 116.3521 97.7132) (end 123.1407 97.7132) (width 0.25) (layer "F.Cu") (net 6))
 (segment (start 123.1407 97.7132) (end 124.4875 99.06) (width 0.25) (layer "F.Cu") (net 6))
 (segment (start 123.1407 95.3118) (end 123.5225 94.93) (width 0.25) (layer "F.Cu") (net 6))
 (segment (start 113.1825 99.3075) (end 114.7578 99.3075) (width 0.25) (layer "F.Cu") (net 6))
 (segment (start 134.6475 104.14) (end 134.6475 99.257) (width 0.25) (layer "F.Cu") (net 10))
 (segment (start 129.5675 109.22) (end 134.6475 104.14) (width 0.25) (layer "F.Cu") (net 10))
 (segment (start 134.6475 99.257) (end 133.35 97.9595) (width 0.25) (layer "F.Cu") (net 10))
 (segment (start 134.6475 104.14) (end 139.7275 109.22) (width 0.25) (layer "F.Cu") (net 10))
 (segment (start 111.6071 104.0668) (end 111.76 104.2197) (width 0.25) (layer "B.Cu") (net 9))
 (segment (start 113.1825 79.8828) (end 111.6071 81.4582) (width 0.25) (layer "B.Cu") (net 9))
 (segment (start 111.6071 81.4582) (end 111.6071 104.0668) (width 0.25) (layer "B.Cu") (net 9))
 (segment (start 113.1825 78.3075) (end 113.1825 79.8828) (width 0.25) (layer "B.Cu") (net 9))
 (segment (start 111.76 105.22) (end 111.76 104.2197) (width 0.25) (layer "B.Cu") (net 9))
 (segment (start 120.2684 105.855) (end 120.5947 106.1813) (width 0.25) (layer "F.Cu") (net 17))
 (segment (start 121.92 106.1813) (end 120.5947 106.1813) (width 0.25) (layer "F.Cu") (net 17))
 (segment (start 116.84 105.855) (end 120.2684 105.855) (width 0.25) (layer "F.Cu") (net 17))
 (segment (start 116.72 111.1797) (end 112.7603 107.22) (width 0.25) (layer "F.Cu") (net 8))
 (segment (start 111.76 107.22) (end 112.7603 107.22) (width 0.25) (layer "F.Cu") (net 8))
 (segment (start 116.84 111.1797) (end 116.72 111.1797) (width 0.25) (layer "F.Cu") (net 8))
 (segment (start 116.84 112.585) (end 116.84 111.1797) (width 0.25) (layer "F.Cu") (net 8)))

